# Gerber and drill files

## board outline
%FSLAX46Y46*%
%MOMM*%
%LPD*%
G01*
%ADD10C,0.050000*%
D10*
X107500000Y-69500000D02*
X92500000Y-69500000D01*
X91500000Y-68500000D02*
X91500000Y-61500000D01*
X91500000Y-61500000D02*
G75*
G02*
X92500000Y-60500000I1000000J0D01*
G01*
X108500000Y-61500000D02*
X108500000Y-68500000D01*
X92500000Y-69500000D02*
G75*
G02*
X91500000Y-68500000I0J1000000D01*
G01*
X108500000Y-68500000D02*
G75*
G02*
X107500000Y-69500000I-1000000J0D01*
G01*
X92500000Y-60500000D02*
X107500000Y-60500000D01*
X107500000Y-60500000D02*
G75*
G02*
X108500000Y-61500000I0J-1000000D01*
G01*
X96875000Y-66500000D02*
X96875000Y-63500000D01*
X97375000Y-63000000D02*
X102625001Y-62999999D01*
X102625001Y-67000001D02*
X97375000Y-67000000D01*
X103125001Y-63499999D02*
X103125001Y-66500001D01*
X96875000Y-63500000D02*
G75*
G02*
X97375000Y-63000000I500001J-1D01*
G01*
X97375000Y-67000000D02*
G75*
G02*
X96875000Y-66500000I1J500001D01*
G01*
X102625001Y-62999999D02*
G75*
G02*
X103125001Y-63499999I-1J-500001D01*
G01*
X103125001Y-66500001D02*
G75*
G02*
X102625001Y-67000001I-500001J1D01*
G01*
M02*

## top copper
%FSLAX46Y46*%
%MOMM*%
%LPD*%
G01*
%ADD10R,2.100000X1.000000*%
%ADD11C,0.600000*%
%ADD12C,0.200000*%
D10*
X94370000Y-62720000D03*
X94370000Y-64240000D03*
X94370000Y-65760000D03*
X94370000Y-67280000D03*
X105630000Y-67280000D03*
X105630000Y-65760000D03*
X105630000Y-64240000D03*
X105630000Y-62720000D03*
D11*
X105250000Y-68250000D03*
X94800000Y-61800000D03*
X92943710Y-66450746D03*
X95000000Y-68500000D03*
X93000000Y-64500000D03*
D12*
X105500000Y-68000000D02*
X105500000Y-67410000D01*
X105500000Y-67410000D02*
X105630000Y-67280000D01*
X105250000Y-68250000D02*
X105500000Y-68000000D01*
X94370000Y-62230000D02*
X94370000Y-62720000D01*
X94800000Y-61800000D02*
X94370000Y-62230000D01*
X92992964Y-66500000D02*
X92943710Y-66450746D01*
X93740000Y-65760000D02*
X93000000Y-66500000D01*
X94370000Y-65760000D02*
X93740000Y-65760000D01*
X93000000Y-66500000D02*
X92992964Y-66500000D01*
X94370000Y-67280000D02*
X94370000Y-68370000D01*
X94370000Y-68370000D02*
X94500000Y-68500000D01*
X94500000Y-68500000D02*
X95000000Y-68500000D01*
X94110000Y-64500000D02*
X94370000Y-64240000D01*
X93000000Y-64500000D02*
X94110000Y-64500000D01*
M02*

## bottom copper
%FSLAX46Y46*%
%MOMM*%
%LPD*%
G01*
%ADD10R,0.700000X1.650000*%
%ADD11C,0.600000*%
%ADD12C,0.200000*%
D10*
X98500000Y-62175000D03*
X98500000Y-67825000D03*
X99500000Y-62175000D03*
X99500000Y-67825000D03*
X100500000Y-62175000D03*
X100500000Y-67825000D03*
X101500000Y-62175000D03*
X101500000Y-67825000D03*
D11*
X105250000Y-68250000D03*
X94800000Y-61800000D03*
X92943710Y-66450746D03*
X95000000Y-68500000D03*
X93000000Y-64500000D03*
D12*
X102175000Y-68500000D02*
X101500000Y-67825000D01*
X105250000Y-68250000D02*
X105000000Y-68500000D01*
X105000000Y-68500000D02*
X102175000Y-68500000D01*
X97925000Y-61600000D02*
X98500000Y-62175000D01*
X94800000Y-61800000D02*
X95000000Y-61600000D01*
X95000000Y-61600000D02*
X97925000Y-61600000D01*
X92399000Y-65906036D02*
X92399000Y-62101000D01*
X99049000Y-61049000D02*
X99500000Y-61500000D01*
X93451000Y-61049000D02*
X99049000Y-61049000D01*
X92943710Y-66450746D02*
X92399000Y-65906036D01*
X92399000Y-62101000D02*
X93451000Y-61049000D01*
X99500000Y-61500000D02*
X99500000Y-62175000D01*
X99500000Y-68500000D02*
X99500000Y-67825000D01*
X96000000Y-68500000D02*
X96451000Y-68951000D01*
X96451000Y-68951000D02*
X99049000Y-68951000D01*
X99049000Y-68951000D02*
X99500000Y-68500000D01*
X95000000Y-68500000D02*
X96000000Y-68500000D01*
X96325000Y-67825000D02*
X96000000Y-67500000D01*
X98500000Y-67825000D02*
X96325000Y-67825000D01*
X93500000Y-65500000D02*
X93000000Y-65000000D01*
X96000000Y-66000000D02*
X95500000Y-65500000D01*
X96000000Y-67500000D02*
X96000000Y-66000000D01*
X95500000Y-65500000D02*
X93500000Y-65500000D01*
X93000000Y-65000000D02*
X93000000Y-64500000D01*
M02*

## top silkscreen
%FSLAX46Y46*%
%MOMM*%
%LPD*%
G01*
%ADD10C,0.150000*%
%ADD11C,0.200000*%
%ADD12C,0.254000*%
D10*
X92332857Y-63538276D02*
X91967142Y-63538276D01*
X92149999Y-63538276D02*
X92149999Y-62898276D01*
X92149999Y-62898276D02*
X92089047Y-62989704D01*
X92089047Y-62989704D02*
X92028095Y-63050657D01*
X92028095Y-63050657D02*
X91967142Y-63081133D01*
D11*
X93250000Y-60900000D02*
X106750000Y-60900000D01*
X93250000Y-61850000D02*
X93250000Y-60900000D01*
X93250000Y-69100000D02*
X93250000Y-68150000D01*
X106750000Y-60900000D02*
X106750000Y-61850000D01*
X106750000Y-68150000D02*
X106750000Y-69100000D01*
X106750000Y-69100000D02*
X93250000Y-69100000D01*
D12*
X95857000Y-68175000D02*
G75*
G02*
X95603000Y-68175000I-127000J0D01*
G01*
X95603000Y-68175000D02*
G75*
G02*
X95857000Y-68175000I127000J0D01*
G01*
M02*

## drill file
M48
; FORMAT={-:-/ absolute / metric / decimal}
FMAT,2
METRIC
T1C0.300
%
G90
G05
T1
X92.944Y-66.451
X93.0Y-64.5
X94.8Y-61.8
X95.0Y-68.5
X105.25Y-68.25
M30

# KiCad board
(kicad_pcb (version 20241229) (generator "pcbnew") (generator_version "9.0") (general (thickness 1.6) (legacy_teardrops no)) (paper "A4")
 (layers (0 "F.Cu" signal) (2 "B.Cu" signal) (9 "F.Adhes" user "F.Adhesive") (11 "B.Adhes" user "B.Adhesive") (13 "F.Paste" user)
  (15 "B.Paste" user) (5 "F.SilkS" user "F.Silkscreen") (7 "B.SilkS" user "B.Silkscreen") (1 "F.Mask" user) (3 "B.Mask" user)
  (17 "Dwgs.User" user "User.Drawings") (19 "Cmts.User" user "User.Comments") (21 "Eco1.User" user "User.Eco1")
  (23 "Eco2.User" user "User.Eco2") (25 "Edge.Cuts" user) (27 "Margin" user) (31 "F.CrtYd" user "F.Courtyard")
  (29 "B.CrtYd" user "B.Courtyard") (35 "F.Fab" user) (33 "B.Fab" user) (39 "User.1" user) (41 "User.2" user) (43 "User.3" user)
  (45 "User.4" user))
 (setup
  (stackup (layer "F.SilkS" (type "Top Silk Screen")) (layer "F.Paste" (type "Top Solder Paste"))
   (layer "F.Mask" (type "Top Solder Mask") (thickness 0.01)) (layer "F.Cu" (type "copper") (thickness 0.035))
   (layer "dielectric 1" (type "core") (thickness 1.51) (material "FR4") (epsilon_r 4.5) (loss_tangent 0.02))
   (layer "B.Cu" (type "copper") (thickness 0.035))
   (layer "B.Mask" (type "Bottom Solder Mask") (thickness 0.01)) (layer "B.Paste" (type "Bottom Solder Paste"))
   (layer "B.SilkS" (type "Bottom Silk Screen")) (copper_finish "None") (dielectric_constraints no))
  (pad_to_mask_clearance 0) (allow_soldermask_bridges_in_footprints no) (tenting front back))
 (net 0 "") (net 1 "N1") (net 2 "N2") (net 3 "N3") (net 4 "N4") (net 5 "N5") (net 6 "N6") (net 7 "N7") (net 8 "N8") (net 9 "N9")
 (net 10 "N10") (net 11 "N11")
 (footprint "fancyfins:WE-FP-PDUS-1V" (layer "F.Cu") (at 100 65)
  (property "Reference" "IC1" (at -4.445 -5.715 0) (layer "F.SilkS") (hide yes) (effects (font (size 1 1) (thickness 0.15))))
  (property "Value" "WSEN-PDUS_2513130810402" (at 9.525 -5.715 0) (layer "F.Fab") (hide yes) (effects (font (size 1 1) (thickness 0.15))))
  (fp_line (start -6.75 -4.1) (end 6.75 -4.1) (stroke (width 0.2) (type solid)) (layer "F.SilkS"))
  (fp_line (start -6.75 -3.15) (end -6.75 -4.1) (stroke (width 0.2) (type solid)) (layer "F.SilkS"))
  (fp_line (start -6.75 4.1) (end -6.75 3.15) (stroke (width 0.2) (type solid)) (layer "F.SilkS"))
  (fp_line (start 6.75 -4.1) (end 6.75 -3.15) (stroke (width 0.2) (type solid)) (layer "F.SilkS"))
  (fp_line (start 6.75 3.15) (end 6.75 4.1) (stroke (width 0.2) (type solid)) (layer "F.SilkS"))
  (fp_line (start 6.75 4.1) (end -6.75 4.1) (stroke (width 0.2) (type solid)) (layer "F.SilkS"))
  (fp_circle (center -4.27 3.175) (end -4.143 3.175) (stroke (width 0.254) (type solid)) (fill no) (layer "F.SilkS"))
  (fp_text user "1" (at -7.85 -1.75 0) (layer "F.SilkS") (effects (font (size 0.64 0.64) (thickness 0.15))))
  (pad "1" smd rect (at -5.63 -2.28) (size 2.1 1) (layers "F.Cu" "F.Mask" "F.Paste") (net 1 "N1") (solder_mask_margin 0.102))
  (pad "2" smd rect (at -5.63 -0.76) (size 2.1 1) (layers "F.Cu" "F.Mask" "F.Paste") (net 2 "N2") (solder_mask_margin 0.102))
  (pad "3" smd rect (at -5.63 0.76) (size 2.1 1) (layers "F.Cu" "F.Mask" "F.Paste") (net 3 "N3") (solder_mask_margin 0.102))
  (pad "4" smd rect (at -5.63 2.28) (size 2.1 1) (layers "F.Cu" "F.Mask" "F.Paste") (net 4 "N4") (solder_mask_margin 0.102))
  (pad "5" smd rect (at 5.63 2.28) (size 2.1 1) (layers "F.Cu" "F.Mask" "F.Paste") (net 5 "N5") (solder_mask_margin 0.102))
  (pad "6" smd rect (at 5.63 0.76) (size 2.1 1) (layers "F.Cu" "F.Mask" "F.Paste") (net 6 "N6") (solder_mask_margin 0.102))
  (pad "7" smd rect (at 5.63 -0.76) (size 2.1 1) (layers "F.Cu" "F.Mask" "F.Paste") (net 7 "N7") (solder_mask_margin 0.102))
  (pad "8" smd rect (at 5.63 -2.28) (size 2.1 1) (layers "F.Cu" "F.Mask" "F.Paste") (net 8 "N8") (solder_mask_margin 0.102))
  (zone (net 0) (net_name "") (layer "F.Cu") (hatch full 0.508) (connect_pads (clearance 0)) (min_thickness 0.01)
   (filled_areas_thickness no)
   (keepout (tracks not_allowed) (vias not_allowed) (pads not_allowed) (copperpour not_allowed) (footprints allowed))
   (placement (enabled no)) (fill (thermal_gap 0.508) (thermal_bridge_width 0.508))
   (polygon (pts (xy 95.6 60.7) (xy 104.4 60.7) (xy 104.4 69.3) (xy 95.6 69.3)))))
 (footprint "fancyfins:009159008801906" (layer "B.Cu") (at 100 65)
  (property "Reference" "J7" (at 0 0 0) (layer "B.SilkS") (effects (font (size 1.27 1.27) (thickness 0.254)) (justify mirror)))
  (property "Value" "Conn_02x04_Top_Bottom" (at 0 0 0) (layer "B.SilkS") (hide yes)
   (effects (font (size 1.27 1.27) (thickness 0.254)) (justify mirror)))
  (fp_line (start -3.125 1.5) (end -3.125 -1.5) (stroke (width 0.05) (type default)) (layer "Edge.Cuts"))
  (fp_line (start -2.625 -2) (end 2.625001 -2.000001) (stroke (width 0.05) (type default)) (layer "Edge.Cuts"))
  (fp_line (start 2.625001 2.000001) (end -2.625 2) (stroke (width 0.05) (type default)) (layer "Edge.Cuts"))
  (fp_line (start 3.125001 -1.500001) (end 3.125001 1.500001) (stroke (width 0.05) (type default)) (layer "Edge.Cuts"))
  (fp_arc (start -3.125 -1.5) (mid -2.978553 -1.853553) (end -2.625 -2) (stroke (width 0.05) (type default)) (layer "Edge.Cuts"))
  (fp_arc (start -2.625 2) (mid -2.978553 1.853553) (end -3.125 1.5) (stroke (width 0.05) (type default)) (layer "Edge.Cuts"))
  (fp_arc (start 2.625001 -2.000001) (mid 2.978554 -1.853554) (end 3.125001 -1.500001) (stroke (width 0.05) (type default))
   (layer "Edge.Cuts"))
  (fp_arc (start 3.125001 1.500001) (mid 2.978554 1.853554) (end 2.625001 2.000001) (stroke (width 0.05) (type default)) (layer "Edge.Cuts"))
  (pad "1" smd rect (at -1.5 -2.825) (size 0.7 1.65) (layers "B.Cu" "B.Mask" "B.Paste") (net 1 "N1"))
  (pad "2" smd rect (at -1.5 2.825) (size 0.7 1.65) (layers "B.Cu" "B.Mask" "B.Paste") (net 2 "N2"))
  (pad "3" smd rect (at -0.5 -2.825) (size 0.7 1.65) (layers "B.Cu" "B.Mask" "B.Paste") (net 3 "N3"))
  (pad "4" smd rect (at -0.5 2.825) (size 0.7 1.65) (layers "B.Cu" "B.Mask" "B.Paste") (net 4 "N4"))
  (pad "5" smd rect (at 0.5 -2.825) (size 0.7 1.65) (layers "B.Cu" "B.Mask" "B.Paste") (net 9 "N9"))
  (pad "6" smd rect (at 0.5 2.825) (size 0.7 1.65) (layers "B.Cu" "B.Mask" "B.Paste") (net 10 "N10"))
  (pad "7" smd rect (at 1.5 -2.825) (size 0.7 1.65) (layers "B.Cu" "B.Mask" "B.Paste") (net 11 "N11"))
  (pad "8" smd rect (at 1.5 2.825) (size 0.7 1.65) (layers "B.Cu" "B.Mask" "B.Paste") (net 5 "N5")))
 (gr_line (start 107.5 69.5) (end 92.5 69.5) (stroke (width 0.05) (type default)) (layer "Edge.Cuts"))
 (gr_line (start 91.5 68.5) (end 91.5 61.5) (stroke (width 0.05) (type default)) (layer "Edge.Cuts"))
 (gr_arc (start 91.5 61.5) (mid 91.792893 60.792893) (end 92.5 60.5) (stroke (width 0.05) (type default)) (layer "Edge.Cuts"))
 (gr_line (start 108.5 61.5) (end 108.5 68.5) (stroke (width 0.05) (type default)) (layer "Edge.Cuts"))
 (gr_arc (start 92.5 69.5) (mid 91.792893 69.207107) (end 91.5 68.5) (stroke (width 0.05) (type default)) (layer "Edge.Cuts"))
 (gr_arc (start 108.5 68.5) (mid 108.207107 69.207107) (end 107.5 69.5) (stroke (width 0.05) (type default)) (layer "Edge.Cuts"))
 (gr_line (start 92.5 60.5) (end 107.5 60.5) (stroke (width 0.05) (type default)) (layer "Edge.Cuts"))
 (gr_arc (start 107.5 60.5) (mid 108.207107 60.792893) (end 108.5 61.5) (stroke (width 0.05) (type default)) (layer "Edge.Cuts"))
 (segment (start 105.5 68) (end 105.5 67.41) (width 0.2) (layer "F.Cu") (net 5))
 (segment (start 105.5 67.41) (end 105.63 67.28) (width 0.2) (layer "F.Cu") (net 5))
 (segment (start 105.25 68.25) (end 105.5 68) (width 0.2) (layer "F.Cu") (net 5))
 (via (at 105.25 68.25) (size 0.6) (drill 0.3) (layers "F.Cu" "B.Cu") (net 5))
 (segment (start 102.175 68.5) (end 101.5 67.825) (width 0.2) (layer "B.Cu") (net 5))
 (segment (start 105.25 68.25) (end 105 68.5) (width 0.2) (layer "B.Cu") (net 5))
 (segment (start 105 68.5) (end 102.175 68.5) (width 0.2) (layer "B.Cu") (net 5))
 (segment (start 94.37 62.23) (end 94.37 62.72) (width 0.2) (layer "F.Cu") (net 1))
 (segment (start 94.8 61.8) (end 94.37 62.23) (width 0.2) (layer "F.Cu") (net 1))
 (via (at 94.8 61.8) (size 0.6) (drill 0.3) (layers "F.Cu" "B.Cu") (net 1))
 (segment (start 97.925 61.6) (end 98.5 62.175) (width 0.2) (layer "B.Cu") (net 1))
 (segment (start 94.8 61.8) (end 95 61.6) (width 0.2) (layer "B.Cu") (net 1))
 (segment (start 95 61.6) (end 97.925 61.6) (width 0.2) (layer "B.Cu") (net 1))
 (segment (start 92.992964 66.5) (end 92.94371 66.450746) (width 0.2) (layer "F.Cu") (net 3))
 (segment (start 93.74 65.76) (end 93 66.5) (width 0.2) (layer "F.Cu") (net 3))
 (segment (start 94.37 65.76) (end 93.74 65.76) (width 0.2) (layer "F.Cu") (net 3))
 (segment (start 93 66.5) (end 92.992964 66.5) (width 0.2) (layer "F.Cu") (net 3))
 (via (at 92.94371 66.450746) (size 0.6) (drill 0.3) (layers "F.Cu" "B.Cu") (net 3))
 (segment (start 92.399 65.906036) (end 92.399 62.101) (width 0.2) (layer "B.Cu") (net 3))
 (segment (start 99.049 61.049) (end 99.5 61.5) (width 0.2) (layer "B.Cu") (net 3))
 (segment (start 93.451 61.049) (end 99.049 61.049) (width 0.2) (layer "B.Cu") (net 3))
 (segment (start 92.94371 66.450746) (end 92.399 65.906036) (width 0.2) (layer "B.Cu") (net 3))
 (segment (start 92.399 62.101) (end 93.451 61.049) (width 0.2) (layer "B.Cu") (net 3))
 (segment (start 99.5 61.5) (end 99.5 62.175) (width 0.2) (layer "B.Cu") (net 3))
 (segment (start 94.37 67.28) (end 94.37 68.37) (width 0.2) (layer "F.Cu") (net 4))
 (segment (start 94.37 68.37) (end 94.5 68.5) (width 0.2) (layer "F.Cu") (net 4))
 (segment (start 94.5 68.5) (end 95 68.5) (width 0.2) (layer "F.Cu") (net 4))
 (via (at 95 68.5) (size 0.6) (drill 0.3) (layers "F.Cu" "B.Cu") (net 4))
 (segment (start 99.5 68.5) (end 99.5 67.825) (width 0.2) (layer "B.Cu") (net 4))
 (segment (start 96 68.5) (end 96.451 68.951) (width 0.2) (layer "B.Cu") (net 4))
 (segment (start 96.451 68.951) (end 99.049 68.951) (width 0.2) (layer "B.Cu") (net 4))
 (segment (start 99.049 68.951) (end 99.5 68.5) (width 0.2) (layer "B.Cu") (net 4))
 (segment (start 95 68.5) (end 96 68.5) (width 0.2) (layer "B.Cu") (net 4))
 (segment (start 94.11 64.5) (end 94.37 64.24) (width 0.2) (layer "F.Cu") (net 2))
 (segment (start 93 64.5) (end 94.11 64.5) (width 0.2) (layer "F.Cu") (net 2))
 (via (at 93 64.5) (size 0.6) (drill 0.3) (layers "F.Cu" "B.Cu") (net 2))
 (segment (start 96.325 67.825) (end 96 67.5) (width 0.2) (layer "B.Cu") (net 2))
 (segment (start 98.5 67.825) (end 96.325 67.825) (width 0.2) (layer "B.Cu") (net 2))
 (segment (start 93.5 65.5) (end 93 65) (width 0.2) (layer "B.Cu") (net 2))
 (segment (start 96 66) (end 95.5 65.5) (width 0.2) (layer "B.Cu") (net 2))
 (segment (start 96 67.5) (end 96 66) (width 0.2) (layer "B.Cu") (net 2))
 (segment (start 95.5 65.5) (end 93.5 65.5) (width 0.2) (layer "B.Cu") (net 2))
 (segment (start 93 65) (end 93 64.5) (width 0.2) (layer "B.Cu") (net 2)))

